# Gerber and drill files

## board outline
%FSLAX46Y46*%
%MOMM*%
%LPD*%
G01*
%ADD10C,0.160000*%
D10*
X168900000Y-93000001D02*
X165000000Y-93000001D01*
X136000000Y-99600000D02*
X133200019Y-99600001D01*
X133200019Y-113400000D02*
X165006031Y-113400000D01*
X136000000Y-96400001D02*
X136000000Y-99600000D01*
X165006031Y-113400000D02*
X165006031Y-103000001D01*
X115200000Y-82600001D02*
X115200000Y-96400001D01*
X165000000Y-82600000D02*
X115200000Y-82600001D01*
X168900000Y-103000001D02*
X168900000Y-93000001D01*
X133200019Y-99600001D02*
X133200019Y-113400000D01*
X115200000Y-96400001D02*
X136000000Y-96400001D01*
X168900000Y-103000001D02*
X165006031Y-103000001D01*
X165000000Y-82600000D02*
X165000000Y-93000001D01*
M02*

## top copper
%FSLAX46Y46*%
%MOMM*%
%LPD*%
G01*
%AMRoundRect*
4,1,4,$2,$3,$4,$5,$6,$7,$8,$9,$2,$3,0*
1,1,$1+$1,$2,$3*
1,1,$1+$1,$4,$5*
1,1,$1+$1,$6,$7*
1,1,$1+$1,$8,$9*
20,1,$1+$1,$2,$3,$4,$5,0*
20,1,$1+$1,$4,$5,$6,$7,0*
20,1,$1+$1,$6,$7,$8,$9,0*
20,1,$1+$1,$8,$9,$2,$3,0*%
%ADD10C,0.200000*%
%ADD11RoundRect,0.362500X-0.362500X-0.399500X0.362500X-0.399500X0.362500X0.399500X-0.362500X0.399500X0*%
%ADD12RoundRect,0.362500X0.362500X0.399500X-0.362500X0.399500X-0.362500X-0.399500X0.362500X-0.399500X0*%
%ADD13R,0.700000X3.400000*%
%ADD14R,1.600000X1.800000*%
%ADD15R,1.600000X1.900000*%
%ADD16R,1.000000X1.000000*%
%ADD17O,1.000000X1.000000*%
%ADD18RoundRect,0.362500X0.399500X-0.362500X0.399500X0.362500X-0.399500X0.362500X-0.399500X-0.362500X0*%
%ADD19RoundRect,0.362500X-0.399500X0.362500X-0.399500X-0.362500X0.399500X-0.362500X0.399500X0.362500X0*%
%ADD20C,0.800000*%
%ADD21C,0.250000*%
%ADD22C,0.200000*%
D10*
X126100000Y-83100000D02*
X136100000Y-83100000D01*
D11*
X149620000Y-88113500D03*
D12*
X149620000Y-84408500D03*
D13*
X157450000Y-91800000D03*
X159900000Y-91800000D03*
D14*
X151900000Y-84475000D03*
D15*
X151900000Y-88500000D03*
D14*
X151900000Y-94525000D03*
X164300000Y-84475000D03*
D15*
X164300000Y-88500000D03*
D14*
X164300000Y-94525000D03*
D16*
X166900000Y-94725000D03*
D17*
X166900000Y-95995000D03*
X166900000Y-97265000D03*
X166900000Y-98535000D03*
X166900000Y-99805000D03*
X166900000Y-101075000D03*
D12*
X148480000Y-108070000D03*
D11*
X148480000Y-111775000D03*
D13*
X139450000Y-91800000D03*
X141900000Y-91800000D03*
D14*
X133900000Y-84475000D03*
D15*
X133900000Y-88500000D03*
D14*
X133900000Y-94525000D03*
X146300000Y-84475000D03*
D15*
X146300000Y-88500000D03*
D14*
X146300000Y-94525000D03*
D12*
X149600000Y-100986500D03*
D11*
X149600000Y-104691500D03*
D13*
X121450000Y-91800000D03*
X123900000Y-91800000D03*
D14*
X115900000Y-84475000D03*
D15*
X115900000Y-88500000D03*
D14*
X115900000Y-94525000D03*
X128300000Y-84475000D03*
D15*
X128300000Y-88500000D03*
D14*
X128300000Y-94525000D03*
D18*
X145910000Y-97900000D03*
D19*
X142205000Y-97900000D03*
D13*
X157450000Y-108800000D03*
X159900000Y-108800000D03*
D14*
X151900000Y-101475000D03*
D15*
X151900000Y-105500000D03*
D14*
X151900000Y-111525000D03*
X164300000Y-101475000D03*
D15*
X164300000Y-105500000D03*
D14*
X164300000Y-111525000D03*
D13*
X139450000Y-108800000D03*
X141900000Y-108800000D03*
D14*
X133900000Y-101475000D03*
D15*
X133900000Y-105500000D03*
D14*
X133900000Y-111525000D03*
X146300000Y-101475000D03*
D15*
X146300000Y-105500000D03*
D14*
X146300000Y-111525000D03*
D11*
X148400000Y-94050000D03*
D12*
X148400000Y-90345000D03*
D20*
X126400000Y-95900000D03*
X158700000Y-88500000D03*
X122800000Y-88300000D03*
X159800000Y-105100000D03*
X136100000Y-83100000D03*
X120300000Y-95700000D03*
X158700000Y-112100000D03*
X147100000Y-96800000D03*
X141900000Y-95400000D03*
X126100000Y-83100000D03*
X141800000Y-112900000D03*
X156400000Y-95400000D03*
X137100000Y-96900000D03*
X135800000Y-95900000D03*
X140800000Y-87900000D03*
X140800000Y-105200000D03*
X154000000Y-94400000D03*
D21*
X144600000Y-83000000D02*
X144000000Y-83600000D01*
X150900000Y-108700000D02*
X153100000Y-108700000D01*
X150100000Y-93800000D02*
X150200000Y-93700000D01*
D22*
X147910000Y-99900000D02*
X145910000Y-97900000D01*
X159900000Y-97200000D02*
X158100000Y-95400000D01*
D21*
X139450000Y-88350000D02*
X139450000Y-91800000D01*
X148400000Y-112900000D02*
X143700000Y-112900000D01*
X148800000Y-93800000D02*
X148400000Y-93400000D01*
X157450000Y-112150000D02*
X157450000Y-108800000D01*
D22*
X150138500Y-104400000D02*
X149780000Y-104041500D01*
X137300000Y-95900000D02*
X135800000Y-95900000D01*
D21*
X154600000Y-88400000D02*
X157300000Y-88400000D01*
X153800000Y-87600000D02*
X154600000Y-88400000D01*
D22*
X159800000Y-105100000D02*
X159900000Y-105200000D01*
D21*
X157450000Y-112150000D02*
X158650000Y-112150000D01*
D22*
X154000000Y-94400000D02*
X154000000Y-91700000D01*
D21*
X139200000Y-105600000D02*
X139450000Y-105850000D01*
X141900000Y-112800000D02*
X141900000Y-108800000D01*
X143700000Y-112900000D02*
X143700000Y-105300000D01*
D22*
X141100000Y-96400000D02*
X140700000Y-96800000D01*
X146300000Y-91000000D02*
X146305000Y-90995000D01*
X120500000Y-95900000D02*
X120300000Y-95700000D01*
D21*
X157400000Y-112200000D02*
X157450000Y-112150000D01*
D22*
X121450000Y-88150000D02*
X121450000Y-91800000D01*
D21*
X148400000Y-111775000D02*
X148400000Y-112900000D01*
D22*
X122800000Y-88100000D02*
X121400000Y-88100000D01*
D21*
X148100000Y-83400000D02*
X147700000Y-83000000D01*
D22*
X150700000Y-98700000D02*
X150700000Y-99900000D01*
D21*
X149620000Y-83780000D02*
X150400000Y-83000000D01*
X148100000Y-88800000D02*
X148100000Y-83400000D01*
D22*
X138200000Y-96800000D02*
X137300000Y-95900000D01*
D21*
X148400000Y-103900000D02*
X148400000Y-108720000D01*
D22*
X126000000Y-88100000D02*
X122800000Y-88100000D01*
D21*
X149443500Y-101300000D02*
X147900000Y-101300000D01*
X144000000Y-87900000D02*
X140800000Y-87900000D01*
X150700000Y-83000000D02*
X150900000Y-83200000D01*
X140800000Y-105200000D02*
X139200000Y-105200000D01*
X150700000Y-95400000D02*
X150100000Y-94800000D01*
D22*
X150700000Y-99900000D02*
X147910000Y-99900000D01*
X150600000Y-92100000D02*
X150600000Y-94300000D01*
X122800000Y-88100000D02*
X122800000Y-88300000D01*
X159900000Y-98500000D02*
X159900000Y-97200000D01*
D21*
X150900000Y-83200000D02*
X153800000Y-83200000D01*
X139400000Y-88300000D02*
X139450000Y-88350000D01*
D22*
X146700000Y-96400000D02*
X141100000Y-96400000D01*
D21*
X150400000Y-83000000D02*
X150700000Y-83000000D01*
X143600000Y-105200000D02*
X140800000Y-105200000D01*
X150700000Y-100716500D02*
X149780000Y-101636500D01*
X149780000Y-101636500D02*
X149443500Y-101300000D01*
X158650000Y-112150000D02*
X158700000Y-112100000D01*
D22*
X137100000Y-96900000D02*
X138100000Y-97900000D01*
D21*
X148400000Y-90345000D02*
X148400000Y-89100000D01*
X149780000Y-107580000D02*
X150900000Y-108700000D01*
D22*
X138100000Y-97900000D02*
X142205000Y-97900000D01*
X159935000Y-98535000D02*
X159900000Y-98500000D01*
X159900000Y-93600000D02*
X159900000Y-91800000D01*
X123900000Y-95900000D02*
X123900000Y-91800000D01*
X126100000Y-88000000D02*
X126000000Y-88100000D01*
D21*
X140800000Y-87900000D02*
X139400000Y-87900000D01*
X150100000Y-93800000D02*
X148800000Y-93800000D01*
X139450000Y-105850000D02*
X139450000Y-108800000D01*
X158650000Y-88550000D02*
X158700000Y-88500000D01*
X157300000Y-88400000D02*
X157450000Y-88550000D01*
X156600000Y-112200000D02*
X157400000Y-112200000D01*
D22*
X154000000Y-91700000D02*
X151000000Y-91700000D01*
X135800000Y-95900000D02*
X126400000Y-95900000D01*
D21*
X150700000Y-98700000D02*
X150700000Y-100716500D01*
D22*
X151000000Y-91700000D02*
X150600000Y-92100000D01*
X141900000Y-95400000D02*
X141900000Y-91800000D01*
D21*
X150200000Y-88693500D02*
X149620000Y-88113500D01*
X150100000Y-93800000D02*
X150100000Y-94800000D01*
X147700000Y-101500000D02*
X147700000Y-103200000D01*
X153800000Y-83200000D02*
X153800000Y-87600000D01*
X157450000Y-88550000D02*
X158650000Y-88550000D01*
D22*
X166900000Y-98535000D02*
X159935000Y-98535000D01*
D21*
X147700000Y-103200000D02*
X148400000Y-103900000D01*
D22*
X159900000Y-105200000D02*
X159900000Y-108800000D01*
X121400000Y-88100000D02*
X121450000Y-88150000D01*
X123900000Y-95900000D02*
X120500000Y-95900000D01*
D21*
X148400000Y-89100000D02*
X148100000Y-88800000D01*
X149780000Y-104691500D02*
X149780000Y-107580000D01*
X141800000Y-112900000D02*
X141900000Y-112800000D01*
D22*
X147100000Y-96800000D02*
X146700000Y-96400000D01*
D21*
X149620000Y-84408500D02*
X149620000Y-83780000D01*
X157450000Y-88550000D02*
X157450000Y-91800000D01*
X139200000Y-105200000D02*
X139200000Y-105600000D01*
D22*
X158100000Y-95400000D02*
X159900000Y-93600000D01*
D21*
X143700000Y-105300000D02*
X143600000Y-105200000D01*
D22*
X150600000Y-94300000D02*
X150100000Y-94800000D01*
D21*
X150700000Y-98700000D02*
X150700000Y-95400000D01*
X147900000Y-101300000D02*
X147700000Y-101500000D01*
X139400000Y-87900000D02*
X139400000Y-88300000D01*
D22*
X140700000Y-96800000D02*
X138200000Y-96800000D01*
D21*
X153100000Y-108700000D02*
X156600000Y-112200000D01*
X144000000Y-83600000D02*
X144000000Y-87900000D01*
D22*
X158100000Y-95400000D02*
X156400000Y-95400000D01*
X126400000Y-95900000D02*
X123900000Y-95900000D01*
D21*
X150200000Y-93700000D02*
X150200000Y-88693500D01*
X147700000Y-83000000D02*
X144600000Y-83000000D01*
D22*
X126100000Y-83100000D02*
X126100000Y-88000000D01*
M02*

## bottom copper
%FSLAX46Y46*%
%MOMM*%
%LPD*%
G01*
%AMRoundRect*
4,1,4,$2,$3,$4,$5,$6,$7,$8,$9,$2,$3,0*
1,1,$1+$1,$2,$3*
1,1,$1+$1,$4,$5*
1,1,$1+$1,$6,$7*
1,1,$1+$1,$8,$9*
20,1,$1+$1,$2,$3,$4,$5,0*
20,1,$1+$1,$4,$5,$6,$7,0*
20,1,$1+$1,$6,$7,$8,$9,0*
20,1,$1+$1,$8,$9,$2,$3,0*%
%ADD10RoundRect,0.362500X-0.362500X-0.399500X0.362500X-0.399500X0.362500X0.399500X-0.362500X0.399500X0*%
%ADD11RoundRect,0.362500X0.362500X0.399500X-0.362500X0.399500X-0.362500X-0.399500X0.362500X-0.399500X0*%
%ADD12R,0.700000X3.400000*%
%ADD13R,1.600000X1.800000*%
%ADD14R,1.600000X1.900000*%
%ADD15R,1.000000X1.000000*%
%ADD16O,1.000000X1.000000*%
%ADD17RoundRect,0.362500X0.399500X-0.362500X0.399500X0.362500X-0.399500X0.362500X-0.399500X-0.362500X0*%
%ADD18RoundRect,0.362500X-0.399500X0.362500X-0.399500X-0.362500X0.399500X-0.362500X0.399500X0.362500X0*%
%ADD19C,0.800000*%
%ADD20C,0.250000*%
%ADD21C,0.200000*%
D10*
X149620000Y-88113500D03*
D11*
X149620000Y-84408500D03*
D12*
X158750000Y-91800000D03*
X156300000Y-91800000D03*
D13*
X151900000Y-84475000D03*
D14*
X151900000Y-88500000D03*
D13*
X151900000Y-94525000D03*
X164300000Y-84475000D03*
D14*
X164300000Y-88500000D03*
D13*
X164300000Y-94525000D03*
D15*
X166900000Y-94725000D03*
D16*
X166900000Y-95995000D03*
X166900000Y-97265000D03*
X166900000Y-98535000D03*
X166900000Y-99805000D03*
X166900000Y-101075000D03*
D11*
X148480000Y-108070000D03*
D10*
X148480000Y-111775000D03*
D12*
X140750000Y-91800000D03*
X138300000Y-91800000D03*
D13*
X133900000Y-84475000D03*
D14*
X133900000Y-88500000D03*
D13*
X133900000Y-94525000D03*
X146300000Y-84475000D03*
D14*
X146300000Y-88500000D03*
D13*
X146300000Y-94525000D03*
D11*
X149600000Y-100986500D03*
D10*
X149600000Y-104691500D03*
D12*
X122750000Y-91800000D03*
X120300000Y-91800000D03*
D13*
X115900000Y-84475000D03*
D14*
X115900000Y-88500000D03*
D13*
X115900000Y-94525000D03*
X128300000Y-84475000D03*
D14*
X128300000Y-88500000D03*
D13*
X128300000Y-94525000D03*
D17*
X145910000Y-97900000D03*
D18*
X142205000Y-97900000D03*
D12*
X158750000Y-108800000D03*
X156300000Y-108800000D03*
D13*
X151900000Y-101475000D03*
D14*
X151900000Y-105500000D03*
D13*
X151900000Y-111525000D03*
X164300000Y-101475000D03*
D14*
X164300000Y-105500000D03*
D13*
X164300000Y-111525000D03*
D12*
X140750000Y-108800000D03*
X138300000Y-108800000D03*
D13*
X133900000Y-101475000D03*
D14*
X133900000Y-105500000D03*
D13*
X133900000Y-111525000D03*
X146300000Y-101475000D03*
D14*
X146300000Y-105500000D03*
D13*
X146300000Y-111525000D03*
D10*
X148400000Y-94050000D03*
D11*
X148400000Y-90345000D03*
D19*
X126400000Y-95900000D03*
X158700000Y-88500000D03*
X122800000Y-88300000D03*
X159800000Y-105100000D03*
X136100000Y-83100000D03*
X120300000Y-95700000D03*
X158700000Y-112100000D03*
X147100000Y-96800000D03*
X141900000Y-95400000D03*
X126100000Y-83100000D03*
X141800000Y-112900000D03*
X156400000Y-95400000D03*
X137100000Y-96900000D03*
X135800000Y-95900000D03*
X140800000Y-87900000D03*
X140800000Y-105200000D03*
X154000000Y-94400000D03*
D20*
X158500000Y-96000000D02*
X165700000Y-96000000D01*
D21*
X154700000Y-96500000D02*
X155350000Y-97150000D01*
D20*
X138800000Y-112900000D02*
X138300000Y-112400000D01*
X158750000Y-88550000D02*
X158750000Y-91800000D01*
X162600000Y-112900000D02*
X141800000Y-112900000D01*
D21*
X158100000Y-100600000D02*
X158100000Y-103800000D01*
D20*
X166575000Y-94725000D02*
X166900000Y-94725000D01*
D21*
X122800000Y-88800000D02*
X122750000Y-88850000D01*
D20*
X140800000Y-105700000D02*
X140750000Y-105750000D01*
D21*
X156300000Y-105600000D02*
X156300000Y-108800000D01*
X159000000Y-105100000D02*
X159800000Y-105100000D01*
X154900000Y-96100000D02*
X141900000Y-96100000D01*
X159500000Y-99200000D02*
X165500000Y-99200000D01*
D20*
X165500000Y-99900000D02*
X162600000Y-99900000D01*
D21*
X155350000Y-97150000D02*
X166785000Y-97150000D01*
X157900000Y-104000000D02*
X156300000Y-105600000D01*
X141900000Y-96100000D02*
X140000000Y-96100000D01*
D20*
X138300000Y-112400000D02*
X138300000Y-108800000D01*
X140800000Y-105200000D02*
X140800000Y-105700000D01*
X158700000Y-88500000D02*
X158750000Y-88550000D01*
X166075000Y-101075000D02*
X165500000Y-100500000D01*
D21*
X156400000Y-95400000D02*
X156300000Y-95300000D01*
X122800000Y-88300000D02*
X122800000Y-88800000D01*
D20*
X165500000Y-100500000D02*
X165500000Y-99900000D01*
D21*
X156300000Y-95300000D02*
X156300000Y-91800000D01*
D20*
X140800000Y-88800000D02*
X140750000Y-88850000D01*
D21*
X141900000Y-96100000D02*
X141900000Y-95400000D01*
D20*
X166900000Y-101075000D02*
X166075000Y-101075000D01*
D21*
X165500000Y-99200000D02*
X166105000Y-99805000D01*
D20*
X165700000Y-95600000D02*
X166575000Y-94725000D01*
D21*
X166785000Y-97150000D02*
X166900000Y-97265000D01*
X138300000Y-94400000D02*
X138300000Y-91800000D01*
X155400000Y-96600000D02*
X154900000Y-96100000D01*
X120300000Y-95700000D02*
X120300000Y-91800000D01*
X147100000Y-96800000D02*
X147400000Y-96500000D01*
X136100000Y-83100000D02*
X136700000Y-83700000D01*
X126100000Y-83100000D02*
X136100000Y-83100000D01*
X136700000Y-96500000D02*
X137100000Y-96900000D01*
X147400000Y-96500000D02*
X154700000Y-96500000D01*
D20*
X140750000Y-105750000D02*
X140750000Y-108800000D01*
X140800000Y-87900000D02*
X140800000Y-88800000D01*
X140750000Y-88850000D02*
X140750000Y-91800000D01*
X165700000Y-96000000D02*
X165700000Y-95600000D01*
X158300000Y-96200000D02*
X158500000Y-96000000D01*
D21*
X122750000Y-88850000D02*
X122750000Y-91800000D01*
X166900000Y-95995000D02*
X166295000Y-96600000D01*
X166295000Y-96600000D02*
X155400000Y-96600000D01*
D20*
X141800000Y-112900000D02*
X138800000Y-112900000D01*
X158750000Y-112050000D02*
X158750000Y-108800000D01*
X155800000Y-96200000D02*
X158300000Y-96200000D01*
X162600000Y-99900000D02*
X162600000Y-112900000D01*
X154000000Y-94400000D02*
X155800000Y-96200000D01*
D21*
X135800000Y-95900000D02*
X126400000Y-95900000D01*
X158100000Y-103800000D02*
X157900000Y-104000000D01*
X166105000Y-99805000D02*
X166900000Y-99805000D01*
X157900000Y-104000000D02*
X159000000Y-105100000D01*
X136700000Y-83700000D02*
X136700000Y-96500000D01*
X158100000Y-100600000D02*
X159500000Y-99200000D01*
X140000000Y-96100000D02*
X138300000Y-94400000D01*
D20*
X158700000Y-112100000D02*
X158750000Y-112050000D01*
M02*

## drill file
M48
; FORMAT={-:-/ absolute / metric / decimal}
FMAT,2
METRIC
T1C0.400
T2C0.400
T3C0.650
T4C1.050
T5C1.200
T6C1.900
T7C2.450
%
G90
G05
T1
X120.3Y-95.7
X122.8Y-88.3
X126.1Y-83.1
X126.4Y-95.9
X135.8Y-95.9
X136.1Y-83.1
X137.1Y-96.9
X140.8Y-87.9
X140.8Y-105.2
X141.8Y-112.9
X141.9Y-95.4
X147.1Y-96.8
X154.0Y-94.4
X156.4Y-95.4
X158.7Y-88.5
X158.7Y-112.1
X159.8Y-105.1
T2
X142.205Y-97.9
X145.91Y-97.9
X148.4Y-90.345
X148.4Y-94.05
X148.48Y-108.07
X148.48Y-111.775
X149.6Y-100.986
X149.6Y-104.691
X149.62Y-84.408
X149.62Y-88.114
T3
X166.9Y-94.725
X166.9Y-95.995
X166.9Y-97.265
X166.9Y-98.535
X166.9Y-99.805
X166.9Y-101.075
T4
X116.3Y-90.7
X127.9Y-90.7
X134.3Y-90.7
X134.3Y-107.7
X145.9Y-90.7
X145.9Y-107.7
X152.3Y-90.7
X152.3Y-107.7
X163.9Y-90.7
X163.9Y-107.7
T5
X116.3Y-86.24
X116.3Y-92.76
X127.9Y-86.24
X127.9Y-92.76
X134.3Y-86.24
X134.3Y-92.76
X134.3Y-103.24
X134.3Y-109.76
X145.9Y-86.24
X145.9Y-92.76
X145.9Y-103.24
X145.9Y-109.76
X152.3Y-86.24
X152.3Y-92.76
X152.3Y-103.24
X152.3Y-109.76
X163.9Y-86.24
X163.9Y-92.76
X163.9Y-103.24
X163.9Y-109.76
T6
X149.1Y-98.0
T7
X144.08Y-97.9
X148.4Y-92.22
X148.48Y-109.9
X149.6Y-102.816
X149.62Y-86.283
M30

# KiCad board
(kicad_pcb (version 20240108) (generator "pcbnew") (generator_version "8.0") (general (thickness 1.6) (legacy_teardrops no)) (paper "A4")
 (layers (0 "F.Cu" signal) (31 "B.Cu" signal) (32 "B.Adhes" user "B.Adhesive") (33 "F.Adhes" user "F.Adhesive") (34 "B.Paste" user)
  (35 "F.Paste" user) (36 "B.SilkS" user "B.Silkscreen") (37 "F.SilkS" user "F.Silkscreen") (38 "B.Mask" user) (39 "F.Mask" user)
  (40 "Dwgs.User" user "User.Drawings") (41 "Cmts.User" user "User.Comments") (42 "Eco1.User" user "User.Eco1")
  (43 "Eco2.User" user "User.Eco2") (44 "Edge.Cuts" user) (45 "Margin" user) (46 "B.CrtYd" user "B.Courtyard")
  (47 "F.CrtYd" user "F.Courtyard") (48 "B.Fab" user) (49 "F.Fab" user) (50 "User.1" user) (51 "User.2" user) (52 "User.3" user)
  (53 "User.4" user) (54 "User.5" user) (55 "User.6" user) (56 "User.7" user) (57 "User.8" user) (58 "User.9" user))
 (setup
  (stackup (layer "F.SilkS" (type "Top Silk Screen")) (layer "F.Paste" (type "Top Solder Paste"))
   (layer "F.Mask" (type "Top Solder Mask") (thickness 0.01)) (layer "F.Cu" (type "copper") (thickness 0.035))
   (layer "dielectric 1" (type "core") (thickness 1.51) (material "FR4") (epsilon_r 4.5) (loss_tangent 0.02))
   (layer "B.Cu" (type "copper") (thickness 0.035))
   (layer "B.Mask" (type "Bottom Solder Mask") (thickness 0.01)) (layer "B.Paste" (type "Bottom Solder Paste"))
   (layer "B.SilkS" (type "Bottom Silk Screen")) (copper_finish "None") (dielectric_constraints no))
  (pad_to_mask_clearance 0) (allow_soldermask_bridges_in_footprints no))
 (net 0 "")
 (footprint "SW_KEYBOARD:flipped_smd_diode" (layer "F.Cu") (at 149.62 89.3035)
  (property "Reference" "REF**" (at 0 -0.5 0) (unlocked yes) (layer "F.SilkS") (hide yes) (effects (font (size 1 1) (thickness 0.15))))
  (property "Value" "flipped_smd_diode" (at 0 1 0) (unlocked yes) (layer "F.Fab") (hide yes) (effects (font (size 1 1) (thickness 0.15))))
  (pad "" np_thru_hole circle (at 0 -3.02) (size 2.45 2.45) (drill 2.45) (layers "*.Mask"))
  (pad "0" thru_hole roundrect (at 0 -1.19) (size 1.45 1.524) (drill 0.4) (layers "*.Cu" "*.Mask") (remove_unused_layers no)
   (roundrect_rratio 0.25))
  (pad "1" thru_hole roundrect (at 0 -4.895 180) (size 1.45 1.524) (drill 0.4) (layers "*.Cu" "*.Mask") (remove_unused_layers no)
   (roundrect_rratio 0.25)))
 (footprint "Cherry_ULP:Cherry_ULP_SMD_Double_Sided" (layer "F.Cu") (at 158.1 89.5)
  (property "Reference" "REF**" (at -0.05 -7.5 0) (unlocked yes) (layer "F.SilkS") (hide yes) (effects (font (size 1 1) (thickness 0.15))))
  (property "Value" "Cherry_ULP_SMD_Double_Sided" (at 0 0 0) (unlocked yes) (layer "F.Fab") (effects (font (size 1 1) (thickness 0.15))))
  (pad "" np_thru_hole circle (at -5.8 -3.26) (size 1.2 1.2) (drill 1.2) (layers "F&B.Cu" "*.Mask"))
  (pad "" np_thru_hole circle (at -5.8 1.2) (size 1.05 1.05) (drill 1.05) (layers "F&B.Cu" "*.Mask"))
  (pad "" np_thru_hole circle (at -5.8 3.26) (size 1.2 1.2) (drill 1.2) (layers "F&B.Cu" "*.Mask"))
  (pad "" np_thru_hole circle (at 5.8 -3.26) (size 1.2 1.2) (drill 1.2) (layers "F&B.Cu" "*.Mask"))
  (pad "" np_thru_hole circle (at 5.8 1.2) (size 1.05 1.05) (drill 1.05) (layers "F&B.Cu" "*.Mask"))
  (pad "" np_thru_hole circle (at 5.8 3.26) (size 1.2 1.2) (drill 1.2) (layers "F&B.Cu" "*.Mask"))
  (pad "1" smd rect (at -0.65 2.3) (size 0.7 3.4) (layers "F.Cu" "F.Paste" "F.Mask"))
  (pad "1" smd rect (at 0.65 2.3) (size 0.7 3.4) (layers "B.Cu" "B.Paste" "B.Mask"))
  (pad "2" smd rect (at -1.8 2.3) (size 0.7 3.4) (layers "B.Cu" "B.Paste" "B.Mask"))
  (pad "2" smd rect (at 1.8 2.3) (size 0.7 3.4) (layers "F.Cu" "F.Paste" "F.Mask"))
  (pad "3" smd rect (at -6.2 -5.025) (size 1.6 1.8) (layers "F.Cu" "F.Paste" "F.Mask"))
  (pad "3" smd rect (at -6.2 -5.025) (size 1.6 1.8) (layers "B.Cu" "B.Paste" "B.Mask"))
  (pad "3" smd rect (at -6.2 -1) (size 1.6 1.9) (layers "F.Cu" "F.Paste" "F.Mask"))
  (pad "3" smd rect (at -6.2 -1) (size 1.6 1.9) (layers "B.Cu" "B.Paste" "B.Mask"))
  (pad "3" smd rect (at -6.2 5.025) (size 1.6 1.8) (layers "F.Cu" "F.Paste" "F.Mask"))
  (pad "3" smd rect (at -6.2 5.025) (size 1.6 1.8) (layers "B.Cu" "B.Paste" "B.Mask"))
  (pad "3" smd rect (at 6.2 -5.025) (size 1.6 1.8) (layers "F.Cu" "F.Paste" "F.Mask"))
  (pad "3" smd rect (at 6.2 -5.025) (size 1.6 1.8) (layers "B.Cu" "B.Paste" "B.Mask"))
  (pad "3" smd rect (at 6.2 -1) (size 1.6 1.9) (layers "F.Cu" "F.Paste" "F.Mask"))
  (pad "3" smd rect (at 6.2 -1) (size 1.6 1.9) (layers "B.Cu" "B.Paste" "B.Mask"))
  (pad "3" smd rect (at 6.2 5.025) (size 1.6 1.8) (layers "F.Cu" "F.Paste" "F.Mask"))
  (pad "3" smd rect (at 6.2 5.025) (size 1.6 1.8) (layers "B.Cu" "B.Paste" "B.Mask"))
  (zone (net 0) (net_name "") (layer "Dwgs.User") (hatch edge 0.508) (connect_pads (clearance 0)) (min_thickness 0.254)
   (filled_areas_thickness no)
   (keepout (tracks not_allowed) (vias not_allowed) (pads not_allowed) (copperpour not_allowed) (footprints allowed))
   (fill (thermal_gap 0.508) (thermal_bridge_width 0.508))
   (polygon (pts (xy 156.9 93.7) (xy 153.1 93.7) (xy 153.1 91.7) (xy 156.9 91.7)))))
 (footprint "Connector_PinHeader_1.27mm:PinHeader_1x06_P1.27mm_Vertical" (layer "F.Cu") (at 166.9 94.725)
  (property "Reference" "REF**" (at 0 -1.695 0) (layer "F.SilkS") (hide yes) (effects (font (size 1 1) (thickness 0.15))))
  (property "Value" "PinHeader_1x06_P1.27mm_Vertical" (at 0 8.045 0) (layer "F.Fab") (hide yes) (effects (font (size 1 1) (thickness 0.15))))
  (pad "1" thru_hole rect (at 0 0) (size 1 1) (drill 0.65) (layers "*.Cu" "*.Mask") (remove_unused_layers no))
  (pad "2" thru_hole oval (at 0 1.27) (size 1 1) (drill 0.65) (layers "*.Cu" "*.Mask") (remove_unused_layers no))
  (pad "3" thru_hole oval (at 0 2.54) (size 1 1) (drill 0.65) (layers "*.Cu" "*.Mask") (remove_unused_layers no))
  (pad "4" thru_hole oval (at 0 3.81) (size 1 1) (drill 0.65) (layers "*.Cu" "*.Mask") (remove_unused_layers no))
  (pad "5" thru_hole oval (at 0 5.08) (size 1 1) (drill 0.65) (layers "*.Cu" "*.Mask") (remove_unused_layers no))
  (pad "6" thru_hole oval (at 0 6.35) (size 1 1) (drill 0.65) (layers "*.Cu" "*.Mask") (remove_unused_layers no)))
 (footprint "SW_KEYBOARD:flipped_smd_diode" (layer "F.Cu") (at 148.48 106.88 180)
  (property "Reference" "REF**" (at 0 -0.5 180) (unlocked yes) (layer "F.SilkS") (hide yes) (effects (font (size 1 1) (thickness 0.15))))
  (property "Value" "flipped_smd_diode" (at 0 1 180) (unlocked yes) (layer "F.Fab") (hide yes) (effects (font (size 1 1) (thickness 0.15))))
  (pad "" np_thru_hole circle (at 0 -3.02 180) (size 2.45 2.45) (drill 2.45) (layers "*.Mask"))
  (pad "0" thru_hole roundrect (at 0 -1.19 180) (size 1.45 1.524) (drill 0.4) (layers "*.Cu" "*.Mask") (remove_unused_layers no)
   (roundrect_rratio 0.25))
  (pad "1" thru_hole roundrect (at 0 -4.895) (size 1.45 1.524) (drill 0.4) (layers "*.Cu" "*.Mask") (remove_unused_layers no)
   (roundrect_rratio 0.25)))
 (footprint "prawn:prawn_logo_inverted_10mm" (layer "F.Cu") (at 155.6 97.9)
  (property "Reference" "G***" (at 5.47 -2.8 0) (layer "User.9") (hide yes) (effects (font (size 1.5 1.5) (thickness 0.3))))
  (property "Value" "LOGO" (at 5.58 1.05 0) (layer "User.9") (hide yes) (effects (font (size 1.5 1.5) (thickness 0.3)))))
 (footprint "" (layer "F.Cu") (at 149.1 98)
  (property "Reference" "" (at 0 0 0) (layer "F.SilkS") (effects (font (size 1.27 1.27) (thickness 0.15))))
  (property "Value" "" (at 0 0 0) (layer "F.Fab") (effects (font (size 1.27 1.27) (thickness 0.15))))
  (pad "" np_thru_hole circle (at 0 0) (size 1.9 1.9) (drill 1.9) (layers "F&B.Cu" "*.Mask")))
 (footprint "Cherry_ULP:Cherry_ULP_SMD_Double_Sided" (layer "F.Cu") (at 140.1 89.5)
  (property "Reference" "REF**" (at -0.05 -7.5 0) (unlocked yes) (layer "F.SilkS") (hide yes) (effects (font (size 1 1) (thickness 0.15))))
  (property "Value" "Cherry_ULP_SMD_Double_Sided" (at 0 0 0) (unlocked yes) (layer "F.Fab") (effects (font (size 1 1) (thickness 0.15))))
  (pad "" np_thru_hole circle (at -5.8 -3.26) (size 1.2 1.2) (drill 1.2) (layers "F&B.Cu" "*.Mask"))
  (pad "" np_thru_hole circle (at -5.8 1.2) (size 1.05 1.05) (drill 1.05) (layers "F&B.Cu" "*.Mask"))
  (pad "" np_thru_hole circle (at -5.8 3.26) (size 1.2 1.2) (drill 1.2) (layers "F&B.Cu" "*.Mask"))
  (pad "" np_thru_hole circle (at 5.8 -3.26) (size 1.2 1.2) (drill 1.2) (layers "F&B.Cu" "*.Mask"))
  (pad "" np_thru_hole circle (at 5.8 1.2) (size 1.05 1.05) (drill 1.05) (layers "F&B.Cu" "*.Mask"))
  (pad "" np_thru_hole circle (at 5.8 3.26) (size 1.2 1.2) (drill 1.2) (layers "F&B.Cu" "*.Mask"))
  (pad "1" smd rect (at -0.65 2.3) (size 0.7 3.4) (layers "F.Cu" "F.Paste" "F.Mask"))
  (pad "1" smd rect (at 0.65 2.3) (size 0.7 3.4) (layers "B.Cu" "B.Paste" "B.Mask"))
  (pad "2" smd rect (at -1.8 2.3) (size 0.7 3.4) (layers "B.Cu" "B.Paste" "B.Mask"))
  (pad "2" smd rect (at 1.8 2.3) (size 0.7 3.4) (layers "F.Cu" "F.Paste" "F.Mask"))
  (pad "3" smd rect (at -6.2 -5.025) (size 1.6 1.8) (layers "F.Cu" "F.Paste" "F.Mask"))
  (pad "3" smd rect (at -6.2 -5.025) (size 1.6 1.8) (layers "B.Cu" "B.Paste" "B.Mask"))
  (pad "3" smd rect (at -6.2 -1) (size 1.6 1.9) (layers "F.Cu" "F.Paste" "F.Mask"))
  (pad "3" smd rect (at -6.2 -1) (size 1.6 1.9) (layers "B.Cu" "B.Paste" "B.Mask"))
  (pad "3" smd rect (at -6.2 5.025) (size 1.6 1.8) (layers "F.Cu" "F.Paste" "F.Mask"))
  (pad "3" smd rect (at -6.2 5.025) (size 1.6 1.8) (layers "B.Cu" "B.Paste" "B.Mask"))
  (pad "3" smd rect (at 6.2 -5.025) (size 1.6 1.8) (layers "F.Cu" "F.Paste" "F.Mask"))
  (pad "3" smd rect (at 6.2 -5.025) (size 1.6 1.8) (layers "B.Cu" "B.Paste" "B.Mask"))
  (pad "3" smd rect (at 6.2 -1) (size 1.6 1.9) (layers "F.Cu" "F.Paste" "F.Mask"))
  (pad "3" smd rect (at 6.2 -1) (size 1.6 1.9) (layers "B.Cu" "B.Paste" "B.Mask"))
  (pad "3" smd rect (at 6.2 5.025) (size 1.6 1.8) (layers "F.Cu" "F.Paste" "F.Mask"))
  (pad "3" smd rect (at 6.2 5.025) (size 1.6 1.8) (layers "B.Cu" "B.Paste" "B.Mask"))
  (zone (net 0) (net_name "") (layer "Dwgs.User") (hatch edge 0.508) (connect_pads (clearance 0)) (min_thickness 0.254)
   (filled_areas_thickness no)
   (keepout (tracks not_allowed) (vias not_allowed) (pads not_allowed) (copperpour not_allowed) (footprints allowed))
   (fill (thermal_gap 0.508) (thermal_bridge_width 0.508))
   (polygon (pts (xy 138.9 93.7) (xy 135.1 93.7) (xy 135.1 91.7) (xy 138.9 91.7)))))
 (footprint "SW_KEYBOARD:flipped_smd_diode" (layer "F.Cu") (at 149.6 99.7965 180)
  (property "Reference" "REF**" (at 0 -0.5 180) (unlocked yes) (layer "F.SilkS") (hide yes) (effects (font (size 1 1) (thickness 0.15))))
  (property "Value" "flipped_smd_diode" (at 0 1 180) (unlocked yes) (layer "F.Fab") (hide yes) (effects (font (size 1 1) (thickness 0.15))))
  (pad "" np_thru_hole circle (at 0 -3.02 180) (size 2.45 2.45) (drill 2.45) (layers "*.Mask"))
  (pad "0" thru_hole roundrect (at 0 -1.19 180) (size 1.45 1.524) (drill 0.4) (layers "*.Cu" "*.Mask") (remove_unused_layers no)
   (roundrect_rratio 0.25))
  (pad "1" thru_hole roundrect (at 0 -4.895) (size 1.45 1.524) (drill 0.4) (layers "*.Cu" "*.Mask") (remove_unused_layers no)
   (roundrect_rratio 0.25)))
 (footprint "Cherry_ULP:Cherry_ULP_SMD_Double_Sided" (layer "F.Cu") (at 122.1 89.5)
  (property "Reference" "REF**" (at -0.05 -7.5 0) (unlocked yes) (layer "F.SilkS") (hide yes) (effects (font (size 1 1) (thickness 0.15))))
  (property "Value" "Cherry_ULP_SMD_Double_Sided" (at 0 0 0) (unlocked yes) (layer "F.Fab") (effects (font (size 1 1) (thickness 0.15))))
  (pad "" np_thru_hole circle (at -5.8 -3.26) (size 1.2 1.2) (drill 1.2) (layers "F&B.Cu" "*.Mask"))
  (pad "" np_thru_hole circle (at -5.8 1.2) (size 1.05 1.05) (drill 1.05) (layers "F&B.Cu" "*.Mask"))
  (pad "" np_thru_hole circle (at -5.8 3.26) (size 1.2 1.2) (drill 1.2) (layers "F&B.Cu" "*.Mask"))
  (pad "" np_thru_hole circle (at 5.8 -3.26) (size 1.2 1.2) (drill 1.2) (layers "F&B.Cu" "*.Mask"))
  (pad "" np_thru_hole circle (at 5.8 1.2) (size 1.05 1.05) (drill 1.05) (layers "F&B.Cu" "*.Mask"))
  (pad "" np_thru_hole circle (at 5.8 3.26) (size 1.2 1.2) (drill 1.2) (layers "F&B.Cu" "*.Mask"))
  (pad "1" smd rect (at -0.65 2.3) (size 0.7 3.4) (layers "F.Cu" "F.Paste" "F.Mask"))
  (pad "1" smd rect (at 0.65 2.3) (size 0.7 3.4) (layers "B.Cu" "B.Paste" "B.Mask"))
  (pad "2" smd rect (at -1.8 2.3) (size 0.7 3.4) (layers "B.Cu" "B.Paste" "B.Mask"))
  (pad "2" smd rect (at 1.8 2.3) (size 0.7 3.4) (layers "F.Cu" "F.Paste" "F.Mask"))
  (pad "3" smd rect (at -6.2 -5.025) (size 1.6 1.8) (layers "F.Cu" "F.Paste" "F.Mask"))
  (pad "3" smd rect (at -6.2 -5.025) (size 1.6 1.8) (layers "B.Cu" "B.Paste" "B.Mask"))
  (pad "3" smd rect (at -6.2 -1) (size 1.6 1.9) (layers "F.Cu" "F.Paste" "F.Mask"))
  (pad "3" smd rect (at -6.2 -1) (size 1.6 1.9) (layers "B.Cu" "B.Paste" "B.Mask"))
  (pad "3" smd rect (at -6.2 5.025) (size 1.6 1.8) (layers "F.Cu" "F.Paste" "F.Mask"))
  (pad "3" smd rect (at -6.2 5.025) (size 1.6 1.8) (layers "B.Cu" "B.Paste" "B.Mask"))
  (pad "3" smd rect (at 6.2 -5.025) (size 1.6 1.8) (layers "F.Cu" "F.Paste" "F.Mask"))
  (pad "3" smd rect (at 6.2 -5.025) (size 1.6 1.8) (layers "B.Cu" "B.Paste" "B.Mask"))
  (pad "3" smd rect (at 6.2 -1) (size 1.6 1.9) (layers "F.Cu" "F.Paste" "F.Mask"))
  (pad "3" smd rect (at 6.2 -1) (size 1.6 1.9) (layers "B.Cu" "B.Paste" "B.Mask"))
  (pad "3" smd rect (at 6.2 5.025) (size 1.6 1.8) (layers "F.Cu" "F.Paste" "F.Mask"))
  (pad "3" smd rect (at 6.2 5.025) (size 1.6 1.8) (layers "B.Cu" "B.Paste" "B.Mask"))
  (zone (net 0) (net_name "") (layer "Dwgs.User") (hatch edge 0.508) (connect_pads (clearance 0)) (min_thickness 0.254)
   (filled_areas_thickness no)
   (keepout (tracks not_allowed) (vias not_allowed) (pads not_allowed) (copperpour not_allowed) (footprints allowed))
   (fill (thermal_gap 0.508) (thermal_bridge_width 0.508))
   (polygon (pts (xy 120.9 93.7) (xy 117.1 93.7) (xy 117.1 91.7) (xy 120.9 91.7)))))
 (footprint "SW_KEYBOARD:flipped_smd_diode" (layer "F.Cu") (at 147.1 97.9 90)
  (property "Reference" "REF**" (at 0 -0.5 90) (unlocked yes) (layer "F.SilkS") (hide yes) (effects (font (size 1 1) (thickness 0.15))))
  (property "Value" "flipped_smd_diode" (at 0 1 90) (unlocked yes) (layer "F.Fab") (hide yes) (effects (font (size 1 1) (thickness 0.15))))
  (pad "" np_thru_hole circle (at 0 -3.02 90) (size 2.45 2.45) (drill 2.45) (layers "*.Mask"))
  (pad "0" thru_hole roundrect (at 0 -1.19 90) (size 1.45 1.524) (drill 0.4) (layers "*.Cu" "*.Mask") (remove_unused_layers no)
   (roundrect_rratio 0.25))
  (pad "1" thru_hole roundrect (at 0 -4.895 270) (size 1.45 1.524) (drill 0.4) (layers "*.Cu" "*.Mask") (remove_unused_layers no)
   (roundrect_rratio 0.25)))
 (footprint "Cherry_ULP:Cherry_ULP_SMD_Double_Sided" (layer "F.Cu") (at 158.1 106.5)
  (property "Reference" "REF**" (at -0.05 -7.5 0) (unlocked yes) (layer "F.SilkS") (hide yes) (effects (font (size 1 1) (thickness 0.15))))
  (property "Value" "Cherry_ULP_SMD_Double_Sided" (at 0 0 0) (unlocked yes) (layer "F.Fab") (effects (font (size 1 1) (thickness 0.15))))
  (pad "" np_thru_hole circle (at -5.8 -3.26) (size 1.2 1.2) (drill 1.2) (layers "F&B.Cu" "*.Mask"))
  (pad "" np_thru_hole circle (at -5.8 1.2) (size 1.05 1.05) (drill 1.05) (layers "F&B.Cu" "*.Mask"))
  (pad "" np_thru_hole circle (at -5.8 3.26) (size 1.2 1.2) (drill 1.2) (layers "F&B.Cu" "*.Mask"))
  (pad "" np_thru_hole circle (at 5.8 -3.26) (size 1.2 1.2) (drill 1.2) (layers "F&B.Cu" "*.Mask"))
  (pad "" np_thru_hole circle (at 5.8 1.2) (size 1.05 1.05) (drill 1.05) (layers "F&B.Cu" "*.Mask"))
  (pad "" np_thru_hole circle (at 5.8 3.26) (size 1.2 1.2) (drill 1.2) (layers "F&B.Cu" "*.Mask"))
  (pad "1" smd rect (at -0.65 2.3) (size 0.7 3.4) (layers "F.Cu" "F.Paste" "F.Mask"))
  (pad "1" smd rect (at 0.65 2.3) (size 0.7 3.4) (layers "B.Cu" "B.Paste" "B.Mask"))
  (pad "2" smd rect (at -1.8 2.3) (size 0.7 3.4) (layers "B.Cu" "B.Paste" "B.Mask"))
  (pad "2" smd rect (at 1.8 2.3) (size 0.7 3.4) (layers "F.Cu" "F.Paste" "F.Mask"))
  (pad "3" smd rect (at -6.2 -5.025) (size 1.6 1.8) (layers "F.Cu" "F.Paste" "F.Mask"))
  (pad "3" smd rect (at -6.2 -5.025) (size 1.6 1.8) (layers "B.Cu" "B.Paste" "B.Mask"))
  (pad "3" smd rect (at -6.2 -1) (size 1.6 1.9) (layers "F.Cu" "F.Paste" "F.Mask"))
  (pad "3" smd rect (at -6.2 -1) (size 1.6 1.9) (layers "B.Cu" "B.Paste" "B.Mask"))
  (pad "3" smd rect (at -6.2 5.025) (size 1.6 1.8) (layers "F.Cu" "F.Paste" "F.Mask"))
  (pad "3" smd rect (at -6.2 5.025) (size 1.6 1.8) (layers "B.Cu" "B.Paste" "B.Mask"))
  (pad "3" smd rect (at 6.2 -5.025) (size 1.6 1.8) (layers "F.Cu" "F.Paste" "F.Mask"))
  (pad "3" smd rect (at 6.2 -5.025) (size 1.6 1.8) (layers "B.Cu" "B.Paste" "B.Mask"))
  (pad "3" smd rect (at 6.2 -1) (size 1.6 1.9) (layers "F.Cu" "F.Paste" "F.Mask"))
  (pad "3" smd rect (at 6.2 -1) (size 1.6 1.9) (layers "B.Cu" "B.Paste" "B.Mask"))
  (pad "3" smd rect (at 6.2 5.025) (size 1.6 1.8) (layers "F.Cu" "F.Paste" "F.Mask"))
  (pad "3" smd rect (at 6.2 5.025) (size 1.6 1.8) (layers "B.Cu" "B.Paste" "B.Mask"))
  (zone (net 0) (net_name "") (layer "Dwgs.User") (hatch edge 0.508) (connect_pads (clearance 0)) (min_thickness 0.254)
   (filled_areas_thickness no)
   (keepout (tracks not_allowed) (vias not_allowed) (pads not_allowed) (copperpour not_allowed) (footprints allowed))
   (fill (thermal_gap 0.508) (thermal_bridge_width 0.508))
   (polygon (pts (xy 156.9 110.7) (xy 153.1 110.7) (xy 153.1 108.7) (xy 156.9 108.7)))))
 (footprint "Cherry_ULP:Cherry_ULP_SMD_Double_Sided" (layer "F.Cu") (at 140.1 106.5)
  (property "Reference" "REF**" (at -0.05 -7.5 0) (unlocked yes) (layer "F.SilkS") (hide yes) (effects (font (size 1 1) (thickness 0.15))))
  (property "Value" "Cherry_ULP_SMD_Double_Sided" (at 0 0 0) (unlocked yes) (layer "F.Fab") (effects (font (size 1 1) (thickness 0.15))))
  (pad "" np_thru_hole circle (at -5.8 -3.26) (size 1.2 1.2) (drill 1.2) (layers "F&B.Cu" "*.Mask"))
  (pad "" np_thru_hole circle (at -5.8 1.2) (size 1.05 1.05) (drill 1.05) (layers "F&B.Cu" "*.Mask"))
  (pad "" np_thru_hole circle (at -5.8 3.26) (size 1.2 1.2) (drill 1.2) (layers "F&B.Cu" "*.Mask"))
  (pad "" np_thru_hole circle (at 5.8 -3.26) (size 1.2 1.2) (drill 1.2) (layers "F&B.Cu" "*.Mask"))
  (pad "" np_thru_hole circle (at 5.8 1.2) (size 1.05 1.05) (drill 1.05) (layers "F&B.Cu" "*.Mask"))
  (pad "" np_thru_hole circle (at 5.8 3.26) (size 1.2 1.2) (drill 1.2) (layers "F&B.Cu" "*.Mask"))
  (pad "1" smd rect (at -0.65 2.3) (size 0.7 3.4) (layers "F.Cu" "F.Paste" "F.Mask"))
  (pad "1" smd rect (at 0.65 2.3) (size 0.7 3.4) (layers "B.Cu" "B.Paste" "B.Mask"))
  (pad "2" smd rect (at -1.8 2.3) (size 0.7 3.4) (layers "B.Cu" "B.Paste" "B.Mask"))
  (pad "2" smd rect (at 1.8 2.3) (size 0.7 3.4) (layers "F.Cu" "F.Paste" "F.Mask"))
  (pad "3" smd rect (at -6.2 -5.025) (size 1.6 1.8) (layers "F.Cu" "F.Paste" "F.Mask"))
  (pad "3" smd rect (at -6.2 -5.025) (size 1.6 1.8) (layers "B.Cu" "B.Paste" "B.Mask"))
  (pad "3" smd rect (at -6.2 -1) (size 1.6 1.9) (layers "F.Cu" "F.Paste" "F.Mask"))
  (pad "3" smd rect (at -6.2 -1) (size 1.6 1.9) (layers "B.Cu" "B.Paste" "B.Mask"))
  (pad "3" smd rect (at -6.2 5.025) (size 1.6 1.8) (layers "F.Cu" "F.Paste" "F.Mask"))
  (pad "3" smd rect (at -6.2 5.025) (size 1.6 1.8) (layers "B.Cu" "B.Paste" "B.Mask"))
  (pad "3" smd rect (at 6.2 -5.025) (size 1.6 1.8) (layers "F.Cu" "F.Paste" "F.Mask"))
  (pad "3" smd rect (at 6.2 -5.025) (size 1.6 1.8) (layers "B.Cu" "B.Paste" "B.Mask"))
  (pad "3" smd rect (at 6.2 -1) (size 1.6 1.9) (layers "F.Cu" "F.Paste" "F.Mask"))
  (pad "3" smd rect (at 6.2 -1) (size 1.6 1.9) (layers "B.Cu" "B.Paste" "B.Mask"))
  (pad "3" smd rect (at 6.2 5.025) (size 1.6 1.8) (layers "F.Cu" "F.Paste" "F.Mask"))
  (pad "3" smd rect (at 6.2 5.025) (size 1.6 1.8) (layers "B.Cu" "B.Paste" "B.Mask"))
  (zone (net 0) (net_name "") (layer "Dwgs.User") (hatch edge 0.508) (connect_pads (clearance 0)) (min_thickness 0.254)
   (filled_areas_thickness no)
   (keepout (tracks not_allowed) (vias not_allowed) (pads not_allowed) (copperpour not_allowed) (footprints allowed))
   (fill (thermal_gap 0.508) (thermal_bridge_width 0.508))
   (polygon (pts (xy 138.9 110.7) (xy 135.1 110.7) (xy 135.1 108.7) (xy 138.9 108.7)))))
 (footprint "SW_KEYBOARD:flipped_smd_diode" (layer "F.Cu") (at 148.4 95.24)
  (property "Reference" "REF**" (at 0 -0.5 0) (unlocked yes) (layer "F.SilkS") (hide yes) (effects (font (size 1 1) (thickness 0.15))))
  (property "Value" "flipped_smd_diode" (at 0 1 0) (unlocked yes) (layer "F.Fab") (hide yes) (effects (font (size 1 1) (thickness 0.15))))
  (pad "" np_thru_hole circle (at 0 -3.02) (size 2.45 2.45) (drill 2.45) (layers "*.Mask"))
  (pad "0" thru_hole roundrect (at 0 -1.19) (size 1.45 1.524) (drill 0.4) (layers "*.Cu" "*.Mask") (remove_unused_layers no)
   (roundrect_rratio 0.25))
  (pad "1" thru_hole roundrect (at 0 -4.895 180) (size 1.45 1.524) (drill 0.4) (layers "*.Cu" "*.Mask") (remove_unused_layers no)
   (roundrect_rratio 0.25)))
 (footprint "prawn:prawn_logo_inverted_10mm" (layer "B.Cu") (at 155.6 97.9 180)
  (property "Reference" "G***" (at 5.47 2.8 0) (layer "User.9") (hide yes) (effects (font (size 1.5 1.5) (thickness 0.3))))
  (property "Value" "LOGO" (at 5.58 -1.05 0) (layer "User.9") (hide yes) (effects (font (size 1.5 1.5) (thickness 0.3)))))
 (gr_line (start 126.1 83.1) (end 136.1 83.1) (stroke (width 0.2) (type default)) (layer "F.Cu"))
 (gr_line (start 168.9 93.000001) (end 165 93.000001) (stroke (width 0.16) (type solid)) (layer "Edge.Cuts"))
 (gr_line (start 136 99.6) (end 133.200019 99.600001) (stroke (width 0.16) (type solid)) (layer "Edge.Cuts"))
 (gr_line (start 133.200019 113.4) (end 165.006031 113.4) (stroke (width 0.16) (type solid)) (layer "Edge.Cuts"))
 (gr_line (start 136 96.400001) (end 136 99.6) (stroke (width 0.16) (type solid)) (layer "Edge.Cuts"))
 (gr_line (start 165.006031 113.4) (end 165.006031 103.000001) (stroke (width 0.16) (type solid)) (layer "Edge.Cuts"))
 (gr_line (start 115.2 82.600001) (end 115.2 96.400001) (stroke (width 0.16) (type solid)) (layer "Edge.Cuts"))
 (gr_line (start 165 82.6) (end 115.2 82.600001) (stroke (width 0.16) (type solid)) (layer "Edge.Cuts"))
 (gr_line (start 168.9 103.000001) (end 168.9 93.000001) (stroke (width 0.16) (type solid)) (layer "Edge.Cuts"))
 (gr_line (start 133.200019 99.600001) (end 133.200019 113.4) (stroke (width 0.16) (type solid)) (layer "Edge.Cuts"))
 (gr_line (start 115.2 96.400001) (end 136 96.400001) (stroke (width 0.16) (type solid)) (layer "Edge.Cuts"))
 (gr_line (start 168.9 103.000001) (end 165.006031 103.000001) (stroke (width 0.16) (type solid)) (layer "Edge.Cuts"))
 (gr_line (start 165 82.6) (end 165 93.000001) (stroke (width 0.16) (type solid)) (layer "Edge.Cuts"))
 (segment (start 144.6 83) (end 144 83.6) (width 0.25) (layer "F.Cu") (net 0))
 (segment (start 150.9 108.7) (end 153.1 108.7) (width 0.25) (layer "F.Cu") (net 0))
 (segment (start 150.1 93.8) (end 150.2 93.7) (width 0.25) (layer "F.Cu") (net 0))
 (segment (start 147.91 99.9) (end 145.91 97.9) (width 0.2) (layer "F.Cu") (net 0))
 (segment (start 159.9 97.2) (end 158.1 95.4) (width 0.2) (layer "F.Cu") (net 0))
 (segment (start 139.45 88.35) (end 139.45 91.8) (width 0.25) (layer "F.Cu") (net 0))
 (segment (start 148.4 112.9) (end 143.7 112.9) (width 0.25) (layer "F.Cu") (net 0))
 (segment (start 148.8 93.8) (end 148.4 93.4) (width 0.25) (layer "F.Cu") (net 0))
 (segment (start 157.45 112.15) (end 157.45 108.8) (width 0.25) (layer "F.Cu") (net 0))
 (segment (start 150.1385 104.4) (end 149.78 104.0415) (width 0.2) (layer "F.Cu") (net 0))
 (segment (start 137.3 95.9) (end 135.8 95.9) (width 0.2) (layer "F.Cu") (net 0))
 (segment (start 154.6 88.4) (end 157.3 88.4) (width 0.25) (layer "F.Cu") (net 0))
 (segment (start 153.8 87.6) (end 154.6 88.4) (width 0.25) (layer "F.Cu") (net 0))
 (segment (start 159.8 105.1) (end 159.9 105.2) (width 0.2) (layer "F.Cu") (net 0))
 (segment (start 157.45 112.15) (end 158.65 112.15) (width 0.25) (layer "F.Cu") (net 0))
 (segment (start 154 94.4) (end 154 91.7) (width 0.2) (layer "F.Cu") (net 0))
 (segment (start 139.2 105.6) (end 139.45 105.85) (width 0.25) (layer "F.Cu") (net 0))
 (segment (start 141.9 112.8) (end 141.9 108.8) (width 0.25) (layer "F.Cu") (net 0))
 (segment (start 143.7 112.9) (end 143.7 105.3) (width 0.25) (layer "F.Cu") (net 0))
 (segment (start 141.1 96.4) (end 140.7 96.8) (width 0.2) (layer "F.Cu") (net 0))
 (segment (start 146.3 91) (end 146.305 90.995) (width 0.2) (layer "F.Cu") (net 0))
 (segment (start 120.5 95.9) (end 120.3 95.7) (width 0.2) (layer "F.Cu") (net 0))
 (segment (start 157.4 112.2) (end 157.45 112.15) (width 0.25) (layer "F.Cu") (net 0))
 (segment (start 121.45 88.15) (end 121.45 91.8) (width 0.2) (layer "F.Cu") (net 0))
 (segment (start 148.4 111.775) (end 148.4 112.9) (width 0.25) (layer "F.Cu") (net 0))
 (segment (start 122.8 88.1) (end 121.4 88.1) (width 0.2) (layer "F.Cu") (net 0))
 (segment (start 148.1 83.4) (end 147.7 83) (width 0.25) (layer "F.Cu") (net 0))
 (segment (start 150.7 98.7) (end 150.7 99.9) (width 0.2) (layer "F.Cu") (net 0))
 (segment (start 149.62 83.78) (end 150.4 83) (width 0.25) (layer "F.Cu") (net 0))
 (segment (start 148.1 88.8) (end 148.1 83.4) (width 0.25) (layer "F.Cu") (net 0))
 (segment (start 138.2 96.8) (end 137.3 95.9) (width 0.2) (layer "F.Cu") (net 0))
 (segment (start 148.4 103.9) (end 148.4 108.72) (width 0.25) (layer "F.Cu") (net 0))
 (segment (start 126 88.1) (end 122.8 88.1) (width 0.2) (layer "F.Cu") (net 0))
 (segment (start 149.4435 101.3) (end 147.9 101.3) (width 0.25) (layer "F.Cu") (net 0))
 (segment (start 144 87.9) (end 140.8 87.9) (width 0.25) (layer "F.Cu") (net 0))
 (segment (start 150.7 83) (end 150.9 83.2) (width 0.25) (layer "F.Cu") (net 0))
 (segment (start 140.8 105.2) (end 139.2 105.2) (width 0.25) (layer "F.Cu") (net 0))
 (segment (start 150.7 95.4) (end 150.1 94.8) (width 0.25) (layer "F.Cu") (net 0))
 (segment (start 150.7 99.9) (end 147.91 99.9) (width 0.2) (layer "F.Cu") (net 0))
 (segment (start 150.6 92.1) (end 150.6 94.3) (width 0.2) (layer "F.Cu") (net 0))
 (segment (start 122.8 88.1) (end 122.8 88.3) (width 0.2) (layer "F.Cu") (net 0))
 (segment (start 159.9 98.5) (end 159.9 97.2) (width 0.2) (layer "F.Cu") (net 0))
 (segment (start 150.9 83.2) (end 153.8 83.2) (width 0.25) (layer "F.Cu") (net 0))
 (segment (start 139.4 88.3) (end 139.45 88.35) (width 0.25) (layer "F.Cu") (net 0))
 (segment (start 146.7 96.4) (end 141.1 96.4) (width 0.2) (layer "F.Cu") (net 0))
 (segment (start 150.4 83) (end 150.7 83) (width 0.25) (layer "F.Cu") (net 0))
 (segment (start 143.6 105.2) (end 140.8 105.2) (width 0.25) (layer "F.Cu") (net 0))
 (segment (start 150.7 100.7165) (end 149.78 101.6365) (width 0.25) (layer "F.Cu") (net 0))
 (segment (start 149.78 101.6365) (end 149.4435 101.3) (width 0.25) (layer "F.Cu") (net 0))
 (segment (start 158.65 112.15) (end 158.7 112.1) (width 0.25) (layer "F.Cu") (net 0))
 (segment (start 137.1 96.9) (end 138.1 97.9) (width 0.2) (layer "F.Cu") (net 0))
 (segment (start 148.4 90.345) (end 148.4 89.1) (width 0.25) (layer "F.Cu") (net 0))
 (segment (start 149.78 107.58) (end 150.9 108.7) (width 0.25) (layer "F.Cu") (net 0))
 (segment (start 138.1 97.9) (end 142.205 97.9) (width 0.2) (layer "F.Cu") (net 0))
 (segment (start 159.935 98.535) (end 159.9 98.5) (width 0.2) (layer "F.Cu") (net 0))
 (segment (start 159.9 93.6) (end 159.9 91.8) (width 0.2) (layer "F.Cu") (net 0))
 (segment (start 123.9 95.9) (end 123.9 91.8) (width 0.2) (layer "F.Cu") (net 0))
 (segment (start 126.1 88) (end 126 88.1) (width 0.2) (layer "F.Cu") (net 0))
 (segment (start 140.8 87.9) (end 139.4 87.9) (width 0.25) (layer "F.Cu") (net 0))
 (segment (start 150.1 93.8) (end 148.8 93.8) (width 0.25) (layer "F.Cu") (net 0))
 (segment (start 139.45 105.85) (end 139.45 108.8) (width 0.25) (layer "F.Cu") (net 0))
 (segment (start 158.65 88.55) (end 158.7 88.5) (width 0.25) (layer "F.Cu") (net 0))
 (segment (start 157.3 88.4) (end 157.45 88.55) (width 0.25) (layer "F.Cu") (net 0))
 (segment (start 156.6 112.2) (end 157.4 112.2) (width 0.25) (layer "F.Cu") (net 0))
 (segment (start 154 91.7) (end 151 91.7) (width 0.2) (layer "F.Cu") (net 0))
 (segment (start 135.8 95.9) (end 126.4 95.9) (width 0.2) (layer "F.Cu") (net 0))
 (segment (start 150.7 98.7) (end 150.7 100.7165) (width 0.25) (layer "F.Cu") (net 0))
 (segment (start 151 91.7) (end 150.6 92.1) (width 0.2) (layer "F.Cu") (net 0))
 (segment (start 141.9 95.4) (end 141.9 91.8) (width 0.2) (layer "F.Cu") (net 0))
 (segment (start 150.2 88.6935) (end 149.62 88.1135) (width 0.25) (layer "F.Cu") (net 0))
 (segment (start 150.1 93.8) (end 150.1 94.8) (width 0.25) (layer "F.Cu") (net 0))
 (segment (start 147.7 101.5) (end 147.7 103.2) (width 0.25) (layer "F.Cu") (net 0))
 (segment (start 153.8 83.2) (end 153.8 87.6) (width 0.25) (layer "F.Cu") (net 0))
 (segment (start 157.45 88.55) (end 158.65 88.55) (width 0.25) (layer "F.Cu") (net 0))
 (segment (start 166.9 98.535) (end 159.935 98.535) (width 0.2) (layer "F.Cu") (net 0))
 (segment (start 147.7 103.2) (end 148.4 103.9) (width 0.25) (layer "F.Cu") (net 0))
 (segment (start 159.9 105.2) (end 159.9 108.8) (width 0.2) (layer "F.Cu") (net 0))
 (segment (start 121.4 88.1) (end 121.45 88.15) (width 0.2) (layer "F.Cu") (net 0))
 (segment (start 123.9 95.9) (end 120.5 95.9) (width 0.2) (layer "F.Cu") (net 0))
 (segment (start 148.4 89.1) (end 148.1 88.8) (width 0.25) (layer "F.Cu") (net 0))
 (segment (start 149.78 104.6915) (end 149.78 107.58) (width 0.25) (layer "F.Cu") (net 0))
 (segment (start 141.8 112.9) (end 141.9 112.8) (width 0.25) (layer "F.Cu") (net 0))
 (segment (start 147.1 96.8) (end 146.7 96.4) (width 0.2) (layer "F.Cu") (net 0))
 (segment (start 149.62 84.4085) (end 149.62 83.78) (width 0.25) (layer "F.Cu") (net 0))
 (segment (start 157.45 88.55) (end 157.45 91.8) (width 0.25) (layer "F.Cu") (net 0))
 (segment (start 139.2 105.2) (end 139.2 105.6) (width 0.25) (layer "F.Cu") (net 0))
 (segment (start 158.1 95.4) (end 159.9 93.6) (width 0.2) (layer "F.Cu") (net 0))
 (segment (start 143.7 105.3) (end 143.6 105.2) (width 0.25) (layer "F.Cu") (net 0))
 (segment (start 150.6 94.3) (end 150.1 94.8) (width 0.2) (layer "F.Cu") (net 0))
 (segment (start 150.7 98.7) (end 150.7 95.4) (width 0.25) (layer "F.Cu") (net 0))
 (segment (start 147.9 101.3) (end 147.7 101.5) (width 0.25) (layer "F.Cu") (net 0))
 (segment (start 139.4 87.9) (end 139.4 88.3) (width 0.25) (layer "F.Cu") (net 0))
 (segment (start 140.7 96.8) (end 138.2 96.8) (width 0.2) (layer "F.Cu") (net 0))
 (segment (start 153.1 108.7) (end 156.6 112.2) (width 0.25) (layer "F.Cu") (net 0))
 (segment (start 144 83.6) (end 144 87.9) (width 0.25) (layer "F.Cu") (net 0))
 (segment (start 158.1 95.4) (end 156.4 95.4) (width 0.2) (layer "F.Cu") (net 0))
 (segment (start 126.4 95.9) (end 123.9 95.9) (width 0.2) (layer "F.Cu") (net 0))
 (segment (start 150.2 93.7) (end 150.2 88.6935) (width 0.25) (layer "F.Cu") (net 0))
 (segment (start 147.7 83) (end 144.6 83) (width 0.25) (layer "F.Cu") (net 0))
 (segment (start 126.1 83.1) (end 126.1 88) (width 0.2) (layer "F.Cu") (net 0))
 (via (at 126.4 95.9) (size 0.8) (drill 0.4) (layers "F.Cu" "B.Cu") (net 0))
 (via (at 158.7 88.5) (size 0.8) (drill 0.4) (layers "F.Cu" "B.Cu") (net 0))
 (via (at 122.8 88.3) (size 0.8) (drill 0.4) (layers "F.Cu" "B.Cu") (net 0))
 (via (at 159.8 105.1) (size 0.8) (drill 0.4) (layers "F.Cu" "B.Cu") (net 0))
 (via (at 136.1 83.1) (size 0.8) (drill 0.4) (layers "F.Cu" "B.Cu") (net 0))
 (via (at 120.3 95.7) (size 0.8) (drill 0.4) (layers "F.Cu" "B.Cu") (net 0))
 (via (at 158.7 112.1) (size 0.8) (drill 0.4) (layers "F.Cu" "B.Cu") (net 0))
 (via (at 147.1 96.8) (size 0.8) (drill 0.4) (layers "F.Cu" "B.Cu") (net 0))
 (via (at 141.9 95.4) (size 0.8) (drill 0.4) (layers "F.Cu" "B.Cu") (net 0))
 (via (at 126.1 83.1) (size 0.8) (drill 0.4) (layers "F.Cu" "B.Cu") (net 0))
 (via (at 141.8 112.9) (size 0.8) (drill 0.4) (layers "F.Cu" "B.Cu") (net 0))
 (via (at 156.4 95.4) (size 0.8) (drill 0.4) (layers "F.Cu" "B.Cu") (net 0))
 (via (at 137.1 96.9) (size 0.8) (drill 0.4) (layers "F.Cu" "B.Cu") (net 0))
 (via (at 135.8 95.9) (size 0.8) (drill 0.4) (layers "F.Cu" "B.Cu") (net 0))
 (via (at 140.8 87.9) (size 0.8) (drill 0.4) (layers "F.Cu" "B.Cu") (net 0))
 (via (at 140.8 105.2) (size 0.8) (drill 0.4) (layers "F.Cu" "B.Cu") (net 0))
 (via (at 154 94.4) (size 0.8) (drill 0.4) (layers "F.Cu" "B.Cu") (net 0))
 (segment (start 158.5 96) (end 165.7 96) (width 0.25) (layer "B.Cu") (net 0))
 (segment (start 154.7 96.5) (end 155.35 97.15) (width 0.2) (layer "B.Cu") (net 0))
 (segment (start 138.8 112.9) (end 138.3 112.4) (width 0.25) (layer "B.Cu") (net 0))
 (segment (start 158.75 88.55) (end 158.75 91.8) (width 0.25) (layer "B.Cu") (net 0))
 (segment (start 162.6 112.9) (end 141.8 112.9) (width 0.25) (layer "B.Cu") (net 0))
 (segment (start 158.1 100.6) (end 158.1 103.8) (width 0.2) (layer "B.Cu") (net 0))
 (segment (start 166.575 94.725) (end 166.9 94.725) (width 0.25) (layer "B.Cu") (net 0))
 (segment (start 122.8 88.8) (end 122.75 88.85) (width 0.2) (layer "B.Cu") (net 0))
 (segment (start 140.8 105.7) (end 140.75 105.75) (width 0.25) (layer "B.Cu") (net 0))
 (segment (start 156.3 105.6) (end 156.3 108.8) (width 0.2) (layer "B.Cu") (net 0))
 (segment (start 159 105.1) (end 159.8 105.1) (width 0.2) (layer "B.Cu") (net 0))
 (segment (start 154.9 96.1) (end 141.9 96.1) (width 0.2) (layer "B.Cu") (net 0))
 (segment (start 159.5 99.2) (end 165.5 99.2) (width 0.2) (layer "B.Cu") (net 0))
 (segment (start 165.5 99.9) (end 162.6 99.9) (width 0.25) (layer "B.Cu") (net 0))
 (segment (start 155.35 97.15) (end 166.785 97.15) (width 0.2) (layer "B.Cu") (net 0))
 (segment (start 157.9 104) (end 156.3 105.6) (width 0.2) (layer "B.Cu") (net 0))
 (segment (start 141.9 96.1) (end 140 96.1) (width 0.2) (layer "B.Cu") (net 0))
 (segment (start 138.3 112.4) (end 138.3 108.8) (width 0.25) (layer "B.Cu") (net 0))
 (segment (start 140.8 105.2) (end 140.8 105.7) (width 0.25) (layer "B.Cu") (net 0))
 (segment (start 158.7 88.5) (end 158.75 88.55) (width 0.25) (layer "B.Cu") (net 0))
 (segment (start 166.075 101.075) (end 165.5 100.5) (width 0.25) (layer "B.Cu") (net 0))
 (segment (start 156.4 95.4) (end 156.3 95.3) (width 0.2) (layer "B.Cu") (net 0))
 (segment (start 122.8 88.3) (end 122.8 88.8) (width 0.2) (layer "B.Cu") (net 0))
 (segment (start 165.5 100.5) (end 165.5 99.9) (width 0.25) (layer "B.Cu") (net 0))
 (segment (start 156.3 95.3) (end 156.3 91.8) (width 0.2) (layer "B.Cu") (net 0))
 (segment (start 140.8 88.8) (end 140.75 88.85) (width 0.25) (layer "B.Cu") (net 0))
 (segment (start 141.9 96.1) (end 141.9 95.4) (width 0.2) (layer "B.Cu") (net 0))
 (segment (start 166.9 101.075) (end 166.075 101.075) (width 0.25) (layer "B.Cu") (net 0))
 (segment (start 165.5 99.2) (end 166.105 99.805) (width 0.2) (layer "B.Cu") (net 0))
 (segment (start 165.7 95.6) (end 166.575 94.725) (width 0.25) (layer "B.Cu") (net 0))
 (segment (start 166.785 97.15) (end 166.9 97.265) (width 0.2) (layer "B.Cu") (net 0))
 (segment (start 138.3 94.4) (end 138.3 91.8) (width 0.2) (layer "B.Cu") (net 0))
 (segment (start 155.4 96.6) (end 154.9 96.1) (width 0.2) (layer "B.Cu") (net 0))
 (segment (start 120.3 95.7) (end 120.3 91.8) (width 0.2) (layer "B.Cu") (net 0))
 (segment (start 147.1 96.8) (end 147.4 96.5) (width 0.2) (layer "B.Cu") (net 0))
 (segment (start 136.1 83.1) (end 136.7 83.7) (width 0.2) (layer "B.Cu") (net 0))
 (segment (start 126.1 83.1) (end 136.1 83.1) (width 0.2) (layer "B.Cu") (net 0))
 (segment (start 136.7 96.5) (end 137.1 96.9) (width 0.2) (layer "B.Cu") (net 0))
 (segment (start 147.4 96.5) (end 154.7 96.5) (width 0.2) (layer "B.Cu") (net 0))
 (segment (start 140.75 105.75) (end 140.75 108.8) (width 0.25) (layer "B.Cu") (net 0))
 (segment (start 140.8 87.9) (end 140.8 88.8) (width 0.25) (layer "B.Cu") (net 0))
 (segment (start 140.75 88.85) (end 140.75 91.8) (width 0.25) (layer "B.Cu") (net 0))
 (segment (start 165.7 96) (end 165.7 95.6) (width 0.25) (layer "B.Cu") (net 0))
 (segment (start 158.3 96.2) (end 158.5 96) (width 0.25) (layer "B.Cu") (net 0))
 (segment (start 122.75 88.85) (end 122.75 91.8) (width 0.2) (layer "B.Cu") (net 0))
 (segment (start 166.9 95.995) (end 166.295 96.6) (width 0.2) (layer "B.Cu") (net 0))
 (segment (start 166.295 96.6) (end 155.4 96.6) (width 0.2) (layer "B.Cu") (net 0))
 (segment (start 141.8 112.9) (end 138.8 112.9) (width 0.25) (layer "B.Cu") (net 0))
 (segment (start 158.75 112.05) (end 158.75 108.8) (width 0.25) (layer "B.Cu") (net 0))
 (segment (start 155.8 96.2) (end 158.3 96.2) (width 0.25) (layer "B.Cu") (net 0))
 (segment (start 162.6 99.9) (end 162.6 112.9) (width 0.25) (layer "B.Cu") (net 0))
 (segment (start 154 94.4) (end 155.8 96.2) (width 0.25) (layer "B.Cu") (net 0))
 (segment (start 135.8 95.9) (end 126.4 95.9) (width 0.2) (layer "B.Cu") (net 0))
 (segment (start 158.1 103.8) (end 157.9 104) (width 0.2) (layer "B.Cu") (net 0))
 (segment (start 166.105 99.805) (end 166.9 99.805) (width 0.2) (layer "B.Cu") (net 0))
 (segment (start 157.9 104) (end 159 105.1) (width 0.2) (layer "B.Cu") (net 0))
 (segment (start 136.7 83.7) (end 136.7 96.5) (width 0.2) (layer "B.Cu") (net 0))
 (segment (start 158.1 100.6) (end 159.5 99.2) (width 0.2) (layer "B.Cu") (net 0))
 (segment (start 140 96.1) (end 138.3 94.4) (width 0.2) (layer "B.Cu") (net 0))
 (segment (start 158.7 112.1) (end 158.75 112.05) (width 0.25) (layer "B.Cu") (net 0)))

